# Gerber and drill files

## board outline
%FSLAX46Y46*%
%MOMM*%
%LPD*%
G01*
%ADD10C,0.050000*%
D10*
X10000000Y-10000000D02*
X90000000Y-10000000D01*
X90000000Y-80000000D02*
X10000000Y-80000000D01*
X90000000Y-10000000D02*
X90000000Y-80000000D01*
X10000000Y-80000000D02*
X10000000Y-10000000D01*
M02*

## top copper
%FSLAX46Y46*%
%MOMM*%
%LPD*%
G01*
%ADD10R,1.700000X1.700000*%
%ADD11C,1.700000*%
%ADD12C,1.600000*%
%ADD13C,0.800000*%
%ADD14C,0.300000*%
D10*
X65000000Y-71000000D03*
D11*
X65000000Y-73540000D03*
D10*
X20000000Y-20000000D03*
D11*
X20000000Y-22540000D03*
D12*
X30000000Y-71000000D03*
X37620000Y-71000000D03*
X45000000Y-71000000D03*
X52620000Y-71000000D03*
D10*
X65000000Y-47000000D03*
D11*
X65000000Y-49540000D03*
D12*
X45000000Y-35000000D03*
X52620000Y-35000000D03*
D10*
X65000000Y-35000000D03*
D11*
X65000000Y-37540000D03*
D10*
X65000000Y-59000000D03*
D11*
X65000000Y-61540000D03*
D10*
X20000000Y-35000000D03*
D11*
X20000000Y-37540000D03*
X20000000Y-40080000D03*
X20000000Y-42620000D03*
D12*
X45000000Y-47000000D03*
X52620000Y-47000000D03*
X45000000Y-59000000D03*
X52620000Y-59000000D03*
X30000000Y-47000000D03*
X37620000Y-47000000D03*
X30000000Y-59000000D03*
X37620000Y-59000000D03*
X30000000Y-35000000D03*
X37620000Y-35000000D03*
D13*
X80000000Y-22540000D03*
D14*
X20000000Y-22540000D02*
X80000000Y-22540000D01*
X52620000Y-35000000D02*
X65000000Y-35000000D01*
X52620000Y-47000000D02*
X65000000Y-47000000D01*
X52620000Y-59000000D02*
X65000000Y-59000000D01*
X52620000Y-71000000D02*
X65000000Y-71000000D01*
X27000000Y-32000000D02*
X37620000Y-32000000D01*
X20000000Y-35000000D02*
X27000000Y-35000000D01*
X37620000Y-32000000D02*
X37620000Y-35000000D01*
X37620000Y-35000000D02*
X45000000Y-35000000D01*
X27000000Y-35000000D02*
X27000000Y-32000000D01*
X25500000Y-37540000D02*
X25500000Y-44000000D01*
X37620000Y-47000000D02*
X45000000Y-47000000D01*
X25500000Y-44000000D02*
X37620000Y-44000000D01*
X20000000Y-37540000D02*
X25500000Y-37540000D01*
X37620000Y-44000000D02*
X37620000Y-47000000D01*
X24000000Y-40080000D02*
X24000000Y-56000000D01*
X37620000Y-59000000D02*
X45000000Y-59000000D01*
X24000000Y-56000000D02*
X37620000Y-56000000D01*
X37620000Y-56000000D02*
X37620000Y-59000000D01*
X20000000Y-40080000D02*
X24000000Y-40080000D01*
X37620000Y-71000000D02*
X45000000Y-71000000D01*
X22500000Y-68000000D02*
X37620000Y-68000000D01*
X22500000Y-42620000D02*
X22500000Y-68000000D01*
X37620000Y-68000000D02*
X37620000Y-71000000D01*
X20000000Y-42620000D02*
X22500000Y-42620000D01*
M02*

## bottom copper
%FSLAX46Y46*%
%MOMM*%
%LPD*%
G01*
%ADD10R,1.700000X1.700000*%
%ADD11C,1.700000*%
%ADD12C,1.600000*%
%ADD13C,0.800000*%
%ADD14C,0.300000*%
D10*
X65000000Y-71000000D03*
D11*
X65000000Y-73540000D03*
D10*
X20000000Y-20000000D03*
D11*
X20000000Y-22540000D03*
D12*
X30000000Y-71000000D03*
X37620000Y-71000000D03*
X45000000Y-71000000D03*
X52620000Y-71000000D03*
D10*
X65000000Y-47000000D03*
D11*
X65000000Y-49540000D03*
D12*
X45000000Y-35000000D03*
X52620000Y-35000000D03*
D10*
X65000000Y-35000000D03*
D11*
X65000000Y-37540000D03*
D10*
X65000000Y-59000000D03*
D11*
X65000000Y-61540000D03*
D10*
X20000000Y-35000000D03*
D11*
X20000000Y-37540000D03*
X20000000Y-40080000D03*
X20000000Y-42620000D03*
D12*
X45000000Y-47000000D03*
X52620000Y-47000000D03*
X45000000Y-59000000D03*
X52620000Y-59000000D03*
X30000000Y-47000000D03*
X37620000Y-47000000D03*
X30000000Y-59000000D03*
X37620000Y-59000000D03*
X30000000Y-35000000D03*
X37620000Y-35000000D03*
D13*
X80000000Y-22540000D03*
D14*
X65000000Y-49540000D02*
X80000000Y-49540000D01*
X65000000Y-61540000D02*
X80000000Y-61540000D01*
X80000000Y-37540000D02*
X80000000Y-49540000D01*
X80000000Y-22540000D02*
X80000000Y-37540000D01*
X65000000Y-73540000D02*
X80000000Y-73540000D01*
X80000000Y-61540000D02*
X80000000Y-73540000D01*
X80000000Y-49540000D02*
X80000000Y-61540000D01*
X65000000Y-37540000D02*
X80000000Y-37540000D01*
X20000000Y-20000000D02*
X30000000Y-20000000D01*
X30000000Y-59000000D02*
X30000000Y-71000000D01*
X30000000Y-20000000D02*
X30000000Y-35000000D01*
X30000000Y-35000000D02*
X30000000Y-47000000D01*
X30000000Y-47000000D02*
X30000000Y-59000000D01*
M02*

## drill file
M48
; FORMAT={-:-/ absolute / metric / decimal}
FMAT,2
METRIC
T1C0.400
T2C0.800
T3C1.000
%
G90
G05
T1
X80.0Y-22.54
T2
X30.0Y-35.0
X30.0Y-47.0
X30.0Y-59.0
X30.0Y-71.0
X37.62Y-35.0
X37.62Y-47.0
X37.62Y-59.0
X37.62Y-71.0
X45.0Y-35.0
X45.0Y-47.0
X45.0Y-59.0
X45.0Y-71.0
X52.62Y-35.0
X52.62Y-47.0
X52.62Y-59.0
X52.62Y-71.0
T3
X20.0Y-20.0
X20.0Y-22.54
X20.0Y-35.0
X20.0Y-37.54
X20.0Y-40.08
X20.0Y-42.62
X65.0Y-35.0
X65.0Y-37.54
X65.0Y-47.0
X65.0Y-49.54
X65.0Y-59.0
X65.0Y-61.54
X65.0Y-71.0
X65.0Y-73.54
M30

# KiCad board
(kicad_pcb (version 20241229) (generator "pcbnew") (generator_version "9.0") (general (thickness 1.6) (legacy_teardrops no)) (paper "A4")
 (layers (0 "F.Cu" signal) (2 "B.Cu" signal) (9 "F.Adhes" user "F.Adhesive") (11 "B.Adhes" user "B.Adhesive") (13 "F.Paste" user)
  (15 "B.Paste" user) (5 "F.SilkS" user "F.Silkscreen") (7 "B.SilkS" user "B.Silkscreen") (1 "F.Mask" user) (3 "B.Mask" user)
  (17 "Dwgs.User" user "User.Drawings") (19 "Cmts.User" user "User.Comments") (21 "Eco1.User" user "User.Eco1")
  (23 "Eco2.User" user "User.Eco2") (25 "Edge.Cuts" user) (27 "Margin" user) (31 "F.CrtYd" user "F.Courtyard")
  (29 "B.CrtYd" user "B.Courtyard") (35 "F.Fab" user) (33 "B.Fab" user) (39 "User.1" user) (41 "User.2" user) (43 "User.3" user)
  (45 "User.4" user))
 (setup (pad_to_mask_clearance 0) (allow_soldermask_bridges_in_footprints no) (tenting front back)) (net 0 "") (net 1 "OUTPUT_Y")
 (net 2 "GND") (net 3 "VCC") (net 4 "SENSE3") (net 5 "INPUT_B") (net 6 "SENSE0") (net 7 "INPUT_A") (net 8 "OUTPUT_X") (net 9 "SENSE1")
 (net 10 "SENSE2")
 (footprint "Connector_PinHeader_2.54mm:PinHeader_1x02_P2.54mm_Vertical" (layer "F.Cu") (at 65 71)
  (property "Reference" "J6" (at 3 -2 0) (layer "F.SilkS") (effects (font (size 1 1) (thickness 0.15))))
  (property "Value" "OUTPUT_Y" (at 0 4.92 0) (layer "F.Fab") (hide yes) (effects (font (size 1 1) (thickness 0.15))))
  (pad "1" thru_hole rect (at 0 0) (size 1.7 1.7) (drill 1) (layers "*.Cu" "*.Mask") (remove_unused_layers no) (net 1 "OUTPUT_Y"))
  (pad "2" thru_hole circle (at 0 2.54) (size 1.7 1.7) (drill 1) (layers "*.Cu" "*.Mask") (remove_unused_layers no) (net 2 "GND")))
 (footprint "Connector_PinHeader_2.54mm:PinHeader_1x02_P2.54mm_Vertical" (layer "F.Cu") (at 20 20)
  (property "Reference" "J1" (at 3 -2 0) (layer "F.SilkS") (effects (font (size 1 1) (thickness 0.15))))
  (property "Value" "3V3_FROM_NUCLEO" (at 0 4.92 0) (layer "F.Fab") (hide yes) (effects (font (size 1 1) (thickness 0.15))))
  (pad "1" thru_hole rect (at 0 0) (size 1.7 1.7) (drill 1) (layers "*.Cu" "*.Mask") (remove_unused_layers no) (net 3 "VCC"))
  (pad "2" thru_hole circle (at 0 2.54) (size 1.7 1.7) (drill 1) (layers "*.Cu" "*.Mask") (remove_unused_layers no) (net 2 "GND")))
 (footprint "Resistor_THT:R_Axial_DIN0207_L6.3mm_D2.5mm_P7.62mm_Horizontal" (layer "F.Cu") (at 30 71)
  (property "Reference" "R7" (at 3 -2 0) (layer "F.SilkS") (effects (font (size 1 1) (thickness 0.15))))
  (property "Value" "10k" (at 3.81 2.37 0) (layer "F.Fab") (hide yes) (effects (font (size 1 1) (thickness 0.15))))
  (pad "1" thru_hole circle (at 0 0) (size 1.6 1.6) (drill 0.8) (layers "*.Cu" "*.Mask") (remove_unused_layers no) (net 3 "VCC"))
  (pad "2" thru_hole circle (at 7.62 0) (size 1.6 1.6) (drill 0.8) (layers "*.Cu" "*.Mask") (remove_unused_layers no) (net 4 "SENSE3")))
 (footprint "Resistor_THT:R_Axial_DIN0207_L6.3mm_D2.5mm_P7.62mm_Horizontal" (layer "F.Cu") (at 45 71)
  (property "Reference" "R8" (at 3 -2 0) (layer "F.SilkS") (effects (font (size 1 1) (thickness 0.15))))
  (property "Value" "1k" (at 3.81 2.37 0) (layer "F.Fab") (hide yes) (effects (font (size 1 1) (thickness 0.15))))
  (pad "1" thru_hole circle (at 0 0) (size 1.6 1.6) (drill 0.8) (layers "*.Cu" "*.Mask") (remove_unused_layers no) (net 4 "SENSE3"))
  (pad "2" thru_hole circle (at 7.62 0) (size 1.6 1.6) (drill 0.8) (layers "*.Cu" "*.Mask") (remove_unused_layers no) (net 1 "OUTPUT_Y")))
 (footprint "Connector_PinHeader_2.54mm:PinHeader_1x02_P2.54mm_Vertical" (layer "F.Cu") (at 65 47)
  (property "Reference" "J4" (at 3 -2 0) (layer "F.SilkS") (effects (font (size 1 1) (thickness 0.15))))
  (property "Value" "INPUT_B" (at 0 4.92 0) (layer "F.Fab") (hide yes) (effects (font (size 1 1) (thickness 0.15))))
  (pad "1" thru_hole rect (at 0 0) (size 1.7 1.7) (drill 1) (layers "*.Cu" "*.Mask") (remove_unused_layers no) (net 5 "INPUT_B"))
  (pad "2" thru_hole circle (at 0 2.54) (size 1.7 1.7) (drill 1) (layers "*.Cu" "*.Mask") (remove_unused_layers no) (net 2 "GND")))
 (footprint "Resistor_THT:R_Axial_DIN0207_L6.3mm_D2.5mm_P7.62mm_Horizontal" (layer "F.Cu") (at 45 35)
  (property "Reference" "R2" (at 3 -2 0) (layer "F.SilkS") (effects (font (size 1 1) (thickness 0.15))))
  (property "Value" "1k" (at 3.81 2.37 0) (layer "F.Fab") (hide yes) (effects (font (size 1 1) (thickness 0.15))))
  (pad "1" thru_hole circle (at 0 0) (size 1.6 1.6) (drill 0.8) (layers "*.Cu" "*.Mask") (remove_unused_layers no) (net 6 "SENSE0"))
  (pad "2" thru_hole circle (at 7.62 0) (size 1.6 1.6) (drill 0.8) (layers "*.Cu" "*.Mask") (remove_unused_layers no) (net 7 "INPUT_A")))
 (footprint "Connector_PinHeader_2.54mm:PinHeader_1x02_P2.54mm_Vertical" (layer "F.Cu") (at 65 35)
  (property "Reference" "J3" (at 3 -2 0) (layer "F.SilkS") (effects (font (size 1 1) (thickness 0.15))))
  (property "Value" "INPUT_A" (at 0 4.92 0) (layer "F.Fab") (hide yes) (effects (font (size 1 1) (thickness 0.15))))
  (pad "1" thru_hole rect (at 0 0) (size 1.7 1.7) (drill 1) (layers "*.Cu" "*.Mask") (remove_unused_layers no) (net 7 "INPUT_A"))
  (pad "2" thru_hole circle (at 0 2.54) (size 1.7 1.7) (drill 1) (layers "*.Cu" "*.Mask") (remove_unused_layers no) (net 2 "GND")))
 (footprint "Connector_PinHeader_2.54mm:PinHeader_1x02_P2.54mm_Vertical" (layer "F.Cu") (at 65 59)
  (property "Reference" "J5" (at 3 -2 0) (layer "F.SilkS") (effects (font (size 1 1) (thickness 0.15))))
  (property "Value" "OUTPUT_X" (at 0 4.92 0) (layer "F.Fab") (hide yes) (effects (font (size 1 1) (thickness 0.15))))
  (pad "1" thru_hole rect (at 0 0) (size 1.7 1.7) (drill 1) (layers "*.Cu" "*.Mask") (remove_unused_layers no) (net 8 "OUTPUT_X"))
  (pad "2" thru_hole circle (at 0 2.54) (size 1.7 1.7) (drill 1) (layers "*.Cu" "*.Mask") (remove_unused_layers no) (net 2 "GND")))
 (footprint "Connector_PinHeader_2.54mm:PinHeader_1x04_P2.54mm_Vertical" (layer "F.Cu") (at 20 35)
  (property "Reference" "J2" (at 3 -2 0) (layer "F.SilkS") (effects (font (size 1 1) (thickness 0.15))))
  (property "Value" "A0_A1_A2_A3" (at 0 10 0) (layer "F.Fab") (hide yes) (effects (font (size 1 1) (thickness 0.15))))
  (pad "1" thru_hole rect (at 0 0) (size 1.7 1.7) (drill 1) (layers "*.Cu" "*.Mask") (remove_unused_layers no) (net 6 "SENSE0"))
  (pad "2" thru_hole circle (at 0 2.54) (size 1.7 1.7) (drill 1) (layers "*.Cu" "*.Mask") (remove_unused_layers no) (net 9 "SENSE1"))
  (pad "3" thru_hole circle (at 0 5.08) (size 1.7 1.7) (drill 1) (layers "*.Cu" "*.Mask") (remove_unused_layers no) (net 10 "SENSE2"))
  (pad "4" thru_hole circle (at 0 7.62) (size 1.7 1.7) (drill 1) (layers "*.Cu" "*.Mask") (remove_unused_layers no) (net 4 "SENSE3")))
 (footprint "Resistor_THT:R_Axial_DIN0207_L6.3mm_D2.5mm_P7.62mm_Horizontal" (layer "F.Cu") (at 45 47)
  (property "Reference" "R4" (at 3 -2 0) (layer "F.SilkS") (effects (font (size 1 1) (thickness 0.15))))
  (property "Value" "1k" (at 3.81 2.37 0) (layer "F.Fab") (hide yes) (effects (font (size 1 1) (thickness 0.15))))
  (pad "1" thru_hole circle (at 0 0) (size 1.6 1.6) (drill 0.8) (layers "*.Cu" "*.Mask") (remove_unused_layers no) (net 9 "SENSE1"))
  (pad "2" thru_hole circle (at 7.62 0) (size 1.6 1.6) (drill 0.8) (layers "*.Cu" "*.Mask") (remove_unused_layers no) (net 5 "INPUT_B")))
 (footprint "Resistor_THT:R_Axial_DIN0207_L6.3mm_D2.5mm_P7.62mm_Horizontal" (layer "F.Cu") (at 45 59)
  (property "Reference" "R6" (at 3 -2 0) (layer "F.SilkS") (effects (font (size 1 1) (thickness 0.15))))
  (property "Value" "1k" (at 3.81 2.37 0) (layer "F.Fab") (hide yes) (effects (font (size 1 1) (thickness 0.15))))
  (pad "1" thru_hole circle (at 0 0) (size 1.6 1.6) (drill 0.8) (layers "*.Cu" "*.Mask") (remove_unused_layers no) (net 10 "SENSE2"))
  (pad "2" thru_hole circle (at 7.62 0) (size 1.6 1.6) (drill 0.8) (layers "*.Cu" "*.Mask") (remove_unused_layers no) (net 8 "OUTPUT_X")))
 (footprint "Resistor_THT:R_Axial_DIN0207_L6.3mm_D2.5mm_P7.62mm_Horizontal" (layer "F.Cu") (at 30 47)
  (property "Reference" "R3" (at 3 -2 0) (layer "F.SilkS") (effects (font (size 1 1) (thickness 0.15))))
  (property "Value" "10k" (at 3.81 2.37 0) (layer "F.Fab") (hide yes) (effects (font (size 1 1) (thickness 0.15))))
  (pad "1" thru_hole circle (at 0 0) (size 1.6 1.6) (drill 0.8) (layers "*.Cu" "*.Mask") (remove_unused_layers no) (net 3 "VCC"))
  (pad "2" thru_hole circle (at 7.62 0) (size 1.6 1.6) (drill 0.8) (layers "*.Cu" "*.Mask") (remove_unused_layers no) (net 9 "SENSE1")))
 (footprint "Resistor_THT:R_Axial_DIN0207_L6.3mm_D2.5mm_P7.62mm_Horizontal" (layer "F.Cu") (at 30 59)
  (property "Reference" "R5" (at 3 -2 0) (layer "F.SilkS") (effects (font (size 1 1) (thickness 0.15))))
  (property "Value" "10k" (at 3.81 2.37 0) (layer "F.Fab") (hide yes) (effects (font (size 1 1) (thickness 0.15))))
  (pad "1" thru_hole circle (at 0 0) (size 1.6 1.6) (drill 0.8) (layers "*.Cu" "*.Mask") (remove_unused_layers no) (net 3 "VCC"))
  (pad "2" thru_hole circle (at 7.62 0) (size 1.6 1.6) (drill 0.8) (layers "*.Cu" "*.Mask") (remove_unused_layers no) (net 10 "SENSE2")))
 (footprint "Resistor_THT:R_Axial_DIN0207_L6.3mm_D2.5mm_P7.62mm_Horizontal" (layer "F.Cu") (at 30 35)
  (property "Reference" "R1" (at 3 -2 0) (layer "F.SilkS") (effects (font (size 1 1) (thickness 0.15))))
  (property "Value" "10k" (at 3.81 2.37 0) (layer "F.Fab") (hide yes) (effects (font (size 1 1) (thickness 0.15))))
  (pad "1" thru_hole circle (at 0 0) (size 1.6 1.6) (drill 0.8) (layers "*.Cu" "*.Mask") (remove_unused_layers no) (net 3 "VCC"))
  (pad "2" thru_hole circle (at 7.62 0) (size 1.6 1.6) (drill 0.8) (layers "*.Cu" "*.Mask") (remove_unused_layers no) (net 6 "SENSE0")))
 (gr_line (start 10 10) (end 90 10) (stroke (width 0.05) (type default)) (layer "Edge.Cuts"))
 (gr_line (start 90 80) (end 10 80) (stroke (width 0.05) (type default)) (layer "Edge.Cuts"))
 (gr_line (start 90 10) (end 90 80) (stroke (width 0.05) (type default)) (layer "Edge.Cuts"))
 (gr_line (start 10 80) (end 10 10) (stroke (width 0.05) (type default)) (layer "Edge.Cuts"))
 (segment (start 20 22.54) (end 80 22.54) (width 0.3) (layer "F.Cu") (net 2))
 (via (at 80 22.54) (size 0.8) (drill 0.4) (layers "F.Cu" "B.Cu") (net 2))
 (segment (start 65 49.54) (end 80 49.54) (width 0.3) (layer "B.Cu") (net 2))
 (segment (start 65 61.54) (end 80 61.54) (width 0.3) (layer "B.Cu") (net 2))
 (segment (start 80 37.54) (end 80 49.54) (width 0.3) (layer "B.Cu") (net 2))
 (segment (start 80 22.54) (end 80 37.54) (width 0.3) (layer "B.Cu") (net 2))
 (segment (start 65 73.54) (end 80 73.54) (width 0.3) (layer "B.Cu") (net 2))
 (segment (start 80 61.54) (end 80 73.54) (width 0.3) (layer "B.Cu") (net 2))
 (segment (start 80 49.54) (end 80 61.54) (width 0.3) (layer "B.Cu") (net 2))
 (segment (start 65 37.54) (end 80 37.54) (width 0.3) (layer "B.Cu") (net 2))
 (segment (start 52.62 35) (end 65 35) (width 0.3) (layer "F.Cu") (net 7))
 (segment (start 52.62 47) (end 65 47) (width 0.3) (layer "F.Cu") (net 5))
 (segment (start 52.62 59) (end 65 59) (width 0.3) (layer "F.Cu") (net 8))
 (segment (start 52.62 71) (end 65 71) (width 0.3) (layer "F.Cu") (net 1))
 (segment (start 27 32) (end 37.62 32) (width 0.3) (layer "F.Cu") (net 6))
 (segment (start 20 35) (end 27 35) (width 0.3) (layer "F.Cu") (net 6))
 (segment (start 37.62 32) (end 37.62 35) (width 0.3) (layer "F.Cu") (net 6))
 (segment (start 37.62 35) (end 45 35) (width 0.3) (layer "F.Cu") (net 6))
 (segment (start 27 35) (end 27 32) (width 0.3) (layer "F.Cu") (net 6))
 (segment (start 25.5 37.54) (end 25.5 44) (width 0.3) (layer "F.Cu") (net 9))
 (segment (start 37.62 47) (end 45 47) (width 0.3) (layer "F.Cu") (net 9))
 (segment (start 25.5 44) (end 37.62 44) (width 0.3) (layer "F.Cu") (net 9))
 (segment (start 20 37.54) (end 25.5 37.54) (width 0.3) (layer "F.Cu") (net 9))
 (segment (start 37.62 44) (end 37.62 47) (width 0.3) (layer "F.Cu") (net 9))
 (segment (start 24 40.08) (end 24 56) (width 0.3) (layer "F.Cu") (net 10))
 (segment (start 37.62 59) (end 45 59) (width 0.3) (layer "F.Cu") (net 10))
 (segment (start 24 56) (end 37.62 56) (width 0.3) (layer "F.Cu") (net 10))
 (segment (start 37.62 56) (end 37.62 59) (width 0.3) (layer "F.Cu") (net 10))
 (segment (start 20 40.08) (end 24 40.08) (width 0.3) (layer "F.Cu") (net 10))
 (segment (start 37.62 71) (end 45 71) (width 0.3) (layer "F.Cu") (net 4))
 (segment (start 22.5 68) (end 37.62 68) (width 0.3) (layer "F.Cu") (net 4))
 (segment (start 22.5 42.62) (end 22.5 68) (width 0.3) (layer "F.Cu") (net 4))
 (segment (start 37.62 68) (end 37.62 71) (width 0.3) (layer "F.Cu") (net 4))
 (segment (start 20 42.62) (end 22.5 42.62) (width 0.3) (layer "F.Cu") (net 4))
 (segment (start 20 20) (end 30 20) (width 0.3) (layer "B.Cu") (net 3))
 (segment (start 30 59) (end 30 71) (width 0.3) (layer "B.Cu") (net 3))
 (segment (start 30 20) (end 30 35) (width 0.3) (layer "B.Cu") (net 3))
 (segment (start 30 35) (end 30 47) (width 0.3) (layer "B.Cu") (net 3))
 (segment (start 30 47) (end 30 59) (width 0.3) (layer "B.Cu") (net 3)))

